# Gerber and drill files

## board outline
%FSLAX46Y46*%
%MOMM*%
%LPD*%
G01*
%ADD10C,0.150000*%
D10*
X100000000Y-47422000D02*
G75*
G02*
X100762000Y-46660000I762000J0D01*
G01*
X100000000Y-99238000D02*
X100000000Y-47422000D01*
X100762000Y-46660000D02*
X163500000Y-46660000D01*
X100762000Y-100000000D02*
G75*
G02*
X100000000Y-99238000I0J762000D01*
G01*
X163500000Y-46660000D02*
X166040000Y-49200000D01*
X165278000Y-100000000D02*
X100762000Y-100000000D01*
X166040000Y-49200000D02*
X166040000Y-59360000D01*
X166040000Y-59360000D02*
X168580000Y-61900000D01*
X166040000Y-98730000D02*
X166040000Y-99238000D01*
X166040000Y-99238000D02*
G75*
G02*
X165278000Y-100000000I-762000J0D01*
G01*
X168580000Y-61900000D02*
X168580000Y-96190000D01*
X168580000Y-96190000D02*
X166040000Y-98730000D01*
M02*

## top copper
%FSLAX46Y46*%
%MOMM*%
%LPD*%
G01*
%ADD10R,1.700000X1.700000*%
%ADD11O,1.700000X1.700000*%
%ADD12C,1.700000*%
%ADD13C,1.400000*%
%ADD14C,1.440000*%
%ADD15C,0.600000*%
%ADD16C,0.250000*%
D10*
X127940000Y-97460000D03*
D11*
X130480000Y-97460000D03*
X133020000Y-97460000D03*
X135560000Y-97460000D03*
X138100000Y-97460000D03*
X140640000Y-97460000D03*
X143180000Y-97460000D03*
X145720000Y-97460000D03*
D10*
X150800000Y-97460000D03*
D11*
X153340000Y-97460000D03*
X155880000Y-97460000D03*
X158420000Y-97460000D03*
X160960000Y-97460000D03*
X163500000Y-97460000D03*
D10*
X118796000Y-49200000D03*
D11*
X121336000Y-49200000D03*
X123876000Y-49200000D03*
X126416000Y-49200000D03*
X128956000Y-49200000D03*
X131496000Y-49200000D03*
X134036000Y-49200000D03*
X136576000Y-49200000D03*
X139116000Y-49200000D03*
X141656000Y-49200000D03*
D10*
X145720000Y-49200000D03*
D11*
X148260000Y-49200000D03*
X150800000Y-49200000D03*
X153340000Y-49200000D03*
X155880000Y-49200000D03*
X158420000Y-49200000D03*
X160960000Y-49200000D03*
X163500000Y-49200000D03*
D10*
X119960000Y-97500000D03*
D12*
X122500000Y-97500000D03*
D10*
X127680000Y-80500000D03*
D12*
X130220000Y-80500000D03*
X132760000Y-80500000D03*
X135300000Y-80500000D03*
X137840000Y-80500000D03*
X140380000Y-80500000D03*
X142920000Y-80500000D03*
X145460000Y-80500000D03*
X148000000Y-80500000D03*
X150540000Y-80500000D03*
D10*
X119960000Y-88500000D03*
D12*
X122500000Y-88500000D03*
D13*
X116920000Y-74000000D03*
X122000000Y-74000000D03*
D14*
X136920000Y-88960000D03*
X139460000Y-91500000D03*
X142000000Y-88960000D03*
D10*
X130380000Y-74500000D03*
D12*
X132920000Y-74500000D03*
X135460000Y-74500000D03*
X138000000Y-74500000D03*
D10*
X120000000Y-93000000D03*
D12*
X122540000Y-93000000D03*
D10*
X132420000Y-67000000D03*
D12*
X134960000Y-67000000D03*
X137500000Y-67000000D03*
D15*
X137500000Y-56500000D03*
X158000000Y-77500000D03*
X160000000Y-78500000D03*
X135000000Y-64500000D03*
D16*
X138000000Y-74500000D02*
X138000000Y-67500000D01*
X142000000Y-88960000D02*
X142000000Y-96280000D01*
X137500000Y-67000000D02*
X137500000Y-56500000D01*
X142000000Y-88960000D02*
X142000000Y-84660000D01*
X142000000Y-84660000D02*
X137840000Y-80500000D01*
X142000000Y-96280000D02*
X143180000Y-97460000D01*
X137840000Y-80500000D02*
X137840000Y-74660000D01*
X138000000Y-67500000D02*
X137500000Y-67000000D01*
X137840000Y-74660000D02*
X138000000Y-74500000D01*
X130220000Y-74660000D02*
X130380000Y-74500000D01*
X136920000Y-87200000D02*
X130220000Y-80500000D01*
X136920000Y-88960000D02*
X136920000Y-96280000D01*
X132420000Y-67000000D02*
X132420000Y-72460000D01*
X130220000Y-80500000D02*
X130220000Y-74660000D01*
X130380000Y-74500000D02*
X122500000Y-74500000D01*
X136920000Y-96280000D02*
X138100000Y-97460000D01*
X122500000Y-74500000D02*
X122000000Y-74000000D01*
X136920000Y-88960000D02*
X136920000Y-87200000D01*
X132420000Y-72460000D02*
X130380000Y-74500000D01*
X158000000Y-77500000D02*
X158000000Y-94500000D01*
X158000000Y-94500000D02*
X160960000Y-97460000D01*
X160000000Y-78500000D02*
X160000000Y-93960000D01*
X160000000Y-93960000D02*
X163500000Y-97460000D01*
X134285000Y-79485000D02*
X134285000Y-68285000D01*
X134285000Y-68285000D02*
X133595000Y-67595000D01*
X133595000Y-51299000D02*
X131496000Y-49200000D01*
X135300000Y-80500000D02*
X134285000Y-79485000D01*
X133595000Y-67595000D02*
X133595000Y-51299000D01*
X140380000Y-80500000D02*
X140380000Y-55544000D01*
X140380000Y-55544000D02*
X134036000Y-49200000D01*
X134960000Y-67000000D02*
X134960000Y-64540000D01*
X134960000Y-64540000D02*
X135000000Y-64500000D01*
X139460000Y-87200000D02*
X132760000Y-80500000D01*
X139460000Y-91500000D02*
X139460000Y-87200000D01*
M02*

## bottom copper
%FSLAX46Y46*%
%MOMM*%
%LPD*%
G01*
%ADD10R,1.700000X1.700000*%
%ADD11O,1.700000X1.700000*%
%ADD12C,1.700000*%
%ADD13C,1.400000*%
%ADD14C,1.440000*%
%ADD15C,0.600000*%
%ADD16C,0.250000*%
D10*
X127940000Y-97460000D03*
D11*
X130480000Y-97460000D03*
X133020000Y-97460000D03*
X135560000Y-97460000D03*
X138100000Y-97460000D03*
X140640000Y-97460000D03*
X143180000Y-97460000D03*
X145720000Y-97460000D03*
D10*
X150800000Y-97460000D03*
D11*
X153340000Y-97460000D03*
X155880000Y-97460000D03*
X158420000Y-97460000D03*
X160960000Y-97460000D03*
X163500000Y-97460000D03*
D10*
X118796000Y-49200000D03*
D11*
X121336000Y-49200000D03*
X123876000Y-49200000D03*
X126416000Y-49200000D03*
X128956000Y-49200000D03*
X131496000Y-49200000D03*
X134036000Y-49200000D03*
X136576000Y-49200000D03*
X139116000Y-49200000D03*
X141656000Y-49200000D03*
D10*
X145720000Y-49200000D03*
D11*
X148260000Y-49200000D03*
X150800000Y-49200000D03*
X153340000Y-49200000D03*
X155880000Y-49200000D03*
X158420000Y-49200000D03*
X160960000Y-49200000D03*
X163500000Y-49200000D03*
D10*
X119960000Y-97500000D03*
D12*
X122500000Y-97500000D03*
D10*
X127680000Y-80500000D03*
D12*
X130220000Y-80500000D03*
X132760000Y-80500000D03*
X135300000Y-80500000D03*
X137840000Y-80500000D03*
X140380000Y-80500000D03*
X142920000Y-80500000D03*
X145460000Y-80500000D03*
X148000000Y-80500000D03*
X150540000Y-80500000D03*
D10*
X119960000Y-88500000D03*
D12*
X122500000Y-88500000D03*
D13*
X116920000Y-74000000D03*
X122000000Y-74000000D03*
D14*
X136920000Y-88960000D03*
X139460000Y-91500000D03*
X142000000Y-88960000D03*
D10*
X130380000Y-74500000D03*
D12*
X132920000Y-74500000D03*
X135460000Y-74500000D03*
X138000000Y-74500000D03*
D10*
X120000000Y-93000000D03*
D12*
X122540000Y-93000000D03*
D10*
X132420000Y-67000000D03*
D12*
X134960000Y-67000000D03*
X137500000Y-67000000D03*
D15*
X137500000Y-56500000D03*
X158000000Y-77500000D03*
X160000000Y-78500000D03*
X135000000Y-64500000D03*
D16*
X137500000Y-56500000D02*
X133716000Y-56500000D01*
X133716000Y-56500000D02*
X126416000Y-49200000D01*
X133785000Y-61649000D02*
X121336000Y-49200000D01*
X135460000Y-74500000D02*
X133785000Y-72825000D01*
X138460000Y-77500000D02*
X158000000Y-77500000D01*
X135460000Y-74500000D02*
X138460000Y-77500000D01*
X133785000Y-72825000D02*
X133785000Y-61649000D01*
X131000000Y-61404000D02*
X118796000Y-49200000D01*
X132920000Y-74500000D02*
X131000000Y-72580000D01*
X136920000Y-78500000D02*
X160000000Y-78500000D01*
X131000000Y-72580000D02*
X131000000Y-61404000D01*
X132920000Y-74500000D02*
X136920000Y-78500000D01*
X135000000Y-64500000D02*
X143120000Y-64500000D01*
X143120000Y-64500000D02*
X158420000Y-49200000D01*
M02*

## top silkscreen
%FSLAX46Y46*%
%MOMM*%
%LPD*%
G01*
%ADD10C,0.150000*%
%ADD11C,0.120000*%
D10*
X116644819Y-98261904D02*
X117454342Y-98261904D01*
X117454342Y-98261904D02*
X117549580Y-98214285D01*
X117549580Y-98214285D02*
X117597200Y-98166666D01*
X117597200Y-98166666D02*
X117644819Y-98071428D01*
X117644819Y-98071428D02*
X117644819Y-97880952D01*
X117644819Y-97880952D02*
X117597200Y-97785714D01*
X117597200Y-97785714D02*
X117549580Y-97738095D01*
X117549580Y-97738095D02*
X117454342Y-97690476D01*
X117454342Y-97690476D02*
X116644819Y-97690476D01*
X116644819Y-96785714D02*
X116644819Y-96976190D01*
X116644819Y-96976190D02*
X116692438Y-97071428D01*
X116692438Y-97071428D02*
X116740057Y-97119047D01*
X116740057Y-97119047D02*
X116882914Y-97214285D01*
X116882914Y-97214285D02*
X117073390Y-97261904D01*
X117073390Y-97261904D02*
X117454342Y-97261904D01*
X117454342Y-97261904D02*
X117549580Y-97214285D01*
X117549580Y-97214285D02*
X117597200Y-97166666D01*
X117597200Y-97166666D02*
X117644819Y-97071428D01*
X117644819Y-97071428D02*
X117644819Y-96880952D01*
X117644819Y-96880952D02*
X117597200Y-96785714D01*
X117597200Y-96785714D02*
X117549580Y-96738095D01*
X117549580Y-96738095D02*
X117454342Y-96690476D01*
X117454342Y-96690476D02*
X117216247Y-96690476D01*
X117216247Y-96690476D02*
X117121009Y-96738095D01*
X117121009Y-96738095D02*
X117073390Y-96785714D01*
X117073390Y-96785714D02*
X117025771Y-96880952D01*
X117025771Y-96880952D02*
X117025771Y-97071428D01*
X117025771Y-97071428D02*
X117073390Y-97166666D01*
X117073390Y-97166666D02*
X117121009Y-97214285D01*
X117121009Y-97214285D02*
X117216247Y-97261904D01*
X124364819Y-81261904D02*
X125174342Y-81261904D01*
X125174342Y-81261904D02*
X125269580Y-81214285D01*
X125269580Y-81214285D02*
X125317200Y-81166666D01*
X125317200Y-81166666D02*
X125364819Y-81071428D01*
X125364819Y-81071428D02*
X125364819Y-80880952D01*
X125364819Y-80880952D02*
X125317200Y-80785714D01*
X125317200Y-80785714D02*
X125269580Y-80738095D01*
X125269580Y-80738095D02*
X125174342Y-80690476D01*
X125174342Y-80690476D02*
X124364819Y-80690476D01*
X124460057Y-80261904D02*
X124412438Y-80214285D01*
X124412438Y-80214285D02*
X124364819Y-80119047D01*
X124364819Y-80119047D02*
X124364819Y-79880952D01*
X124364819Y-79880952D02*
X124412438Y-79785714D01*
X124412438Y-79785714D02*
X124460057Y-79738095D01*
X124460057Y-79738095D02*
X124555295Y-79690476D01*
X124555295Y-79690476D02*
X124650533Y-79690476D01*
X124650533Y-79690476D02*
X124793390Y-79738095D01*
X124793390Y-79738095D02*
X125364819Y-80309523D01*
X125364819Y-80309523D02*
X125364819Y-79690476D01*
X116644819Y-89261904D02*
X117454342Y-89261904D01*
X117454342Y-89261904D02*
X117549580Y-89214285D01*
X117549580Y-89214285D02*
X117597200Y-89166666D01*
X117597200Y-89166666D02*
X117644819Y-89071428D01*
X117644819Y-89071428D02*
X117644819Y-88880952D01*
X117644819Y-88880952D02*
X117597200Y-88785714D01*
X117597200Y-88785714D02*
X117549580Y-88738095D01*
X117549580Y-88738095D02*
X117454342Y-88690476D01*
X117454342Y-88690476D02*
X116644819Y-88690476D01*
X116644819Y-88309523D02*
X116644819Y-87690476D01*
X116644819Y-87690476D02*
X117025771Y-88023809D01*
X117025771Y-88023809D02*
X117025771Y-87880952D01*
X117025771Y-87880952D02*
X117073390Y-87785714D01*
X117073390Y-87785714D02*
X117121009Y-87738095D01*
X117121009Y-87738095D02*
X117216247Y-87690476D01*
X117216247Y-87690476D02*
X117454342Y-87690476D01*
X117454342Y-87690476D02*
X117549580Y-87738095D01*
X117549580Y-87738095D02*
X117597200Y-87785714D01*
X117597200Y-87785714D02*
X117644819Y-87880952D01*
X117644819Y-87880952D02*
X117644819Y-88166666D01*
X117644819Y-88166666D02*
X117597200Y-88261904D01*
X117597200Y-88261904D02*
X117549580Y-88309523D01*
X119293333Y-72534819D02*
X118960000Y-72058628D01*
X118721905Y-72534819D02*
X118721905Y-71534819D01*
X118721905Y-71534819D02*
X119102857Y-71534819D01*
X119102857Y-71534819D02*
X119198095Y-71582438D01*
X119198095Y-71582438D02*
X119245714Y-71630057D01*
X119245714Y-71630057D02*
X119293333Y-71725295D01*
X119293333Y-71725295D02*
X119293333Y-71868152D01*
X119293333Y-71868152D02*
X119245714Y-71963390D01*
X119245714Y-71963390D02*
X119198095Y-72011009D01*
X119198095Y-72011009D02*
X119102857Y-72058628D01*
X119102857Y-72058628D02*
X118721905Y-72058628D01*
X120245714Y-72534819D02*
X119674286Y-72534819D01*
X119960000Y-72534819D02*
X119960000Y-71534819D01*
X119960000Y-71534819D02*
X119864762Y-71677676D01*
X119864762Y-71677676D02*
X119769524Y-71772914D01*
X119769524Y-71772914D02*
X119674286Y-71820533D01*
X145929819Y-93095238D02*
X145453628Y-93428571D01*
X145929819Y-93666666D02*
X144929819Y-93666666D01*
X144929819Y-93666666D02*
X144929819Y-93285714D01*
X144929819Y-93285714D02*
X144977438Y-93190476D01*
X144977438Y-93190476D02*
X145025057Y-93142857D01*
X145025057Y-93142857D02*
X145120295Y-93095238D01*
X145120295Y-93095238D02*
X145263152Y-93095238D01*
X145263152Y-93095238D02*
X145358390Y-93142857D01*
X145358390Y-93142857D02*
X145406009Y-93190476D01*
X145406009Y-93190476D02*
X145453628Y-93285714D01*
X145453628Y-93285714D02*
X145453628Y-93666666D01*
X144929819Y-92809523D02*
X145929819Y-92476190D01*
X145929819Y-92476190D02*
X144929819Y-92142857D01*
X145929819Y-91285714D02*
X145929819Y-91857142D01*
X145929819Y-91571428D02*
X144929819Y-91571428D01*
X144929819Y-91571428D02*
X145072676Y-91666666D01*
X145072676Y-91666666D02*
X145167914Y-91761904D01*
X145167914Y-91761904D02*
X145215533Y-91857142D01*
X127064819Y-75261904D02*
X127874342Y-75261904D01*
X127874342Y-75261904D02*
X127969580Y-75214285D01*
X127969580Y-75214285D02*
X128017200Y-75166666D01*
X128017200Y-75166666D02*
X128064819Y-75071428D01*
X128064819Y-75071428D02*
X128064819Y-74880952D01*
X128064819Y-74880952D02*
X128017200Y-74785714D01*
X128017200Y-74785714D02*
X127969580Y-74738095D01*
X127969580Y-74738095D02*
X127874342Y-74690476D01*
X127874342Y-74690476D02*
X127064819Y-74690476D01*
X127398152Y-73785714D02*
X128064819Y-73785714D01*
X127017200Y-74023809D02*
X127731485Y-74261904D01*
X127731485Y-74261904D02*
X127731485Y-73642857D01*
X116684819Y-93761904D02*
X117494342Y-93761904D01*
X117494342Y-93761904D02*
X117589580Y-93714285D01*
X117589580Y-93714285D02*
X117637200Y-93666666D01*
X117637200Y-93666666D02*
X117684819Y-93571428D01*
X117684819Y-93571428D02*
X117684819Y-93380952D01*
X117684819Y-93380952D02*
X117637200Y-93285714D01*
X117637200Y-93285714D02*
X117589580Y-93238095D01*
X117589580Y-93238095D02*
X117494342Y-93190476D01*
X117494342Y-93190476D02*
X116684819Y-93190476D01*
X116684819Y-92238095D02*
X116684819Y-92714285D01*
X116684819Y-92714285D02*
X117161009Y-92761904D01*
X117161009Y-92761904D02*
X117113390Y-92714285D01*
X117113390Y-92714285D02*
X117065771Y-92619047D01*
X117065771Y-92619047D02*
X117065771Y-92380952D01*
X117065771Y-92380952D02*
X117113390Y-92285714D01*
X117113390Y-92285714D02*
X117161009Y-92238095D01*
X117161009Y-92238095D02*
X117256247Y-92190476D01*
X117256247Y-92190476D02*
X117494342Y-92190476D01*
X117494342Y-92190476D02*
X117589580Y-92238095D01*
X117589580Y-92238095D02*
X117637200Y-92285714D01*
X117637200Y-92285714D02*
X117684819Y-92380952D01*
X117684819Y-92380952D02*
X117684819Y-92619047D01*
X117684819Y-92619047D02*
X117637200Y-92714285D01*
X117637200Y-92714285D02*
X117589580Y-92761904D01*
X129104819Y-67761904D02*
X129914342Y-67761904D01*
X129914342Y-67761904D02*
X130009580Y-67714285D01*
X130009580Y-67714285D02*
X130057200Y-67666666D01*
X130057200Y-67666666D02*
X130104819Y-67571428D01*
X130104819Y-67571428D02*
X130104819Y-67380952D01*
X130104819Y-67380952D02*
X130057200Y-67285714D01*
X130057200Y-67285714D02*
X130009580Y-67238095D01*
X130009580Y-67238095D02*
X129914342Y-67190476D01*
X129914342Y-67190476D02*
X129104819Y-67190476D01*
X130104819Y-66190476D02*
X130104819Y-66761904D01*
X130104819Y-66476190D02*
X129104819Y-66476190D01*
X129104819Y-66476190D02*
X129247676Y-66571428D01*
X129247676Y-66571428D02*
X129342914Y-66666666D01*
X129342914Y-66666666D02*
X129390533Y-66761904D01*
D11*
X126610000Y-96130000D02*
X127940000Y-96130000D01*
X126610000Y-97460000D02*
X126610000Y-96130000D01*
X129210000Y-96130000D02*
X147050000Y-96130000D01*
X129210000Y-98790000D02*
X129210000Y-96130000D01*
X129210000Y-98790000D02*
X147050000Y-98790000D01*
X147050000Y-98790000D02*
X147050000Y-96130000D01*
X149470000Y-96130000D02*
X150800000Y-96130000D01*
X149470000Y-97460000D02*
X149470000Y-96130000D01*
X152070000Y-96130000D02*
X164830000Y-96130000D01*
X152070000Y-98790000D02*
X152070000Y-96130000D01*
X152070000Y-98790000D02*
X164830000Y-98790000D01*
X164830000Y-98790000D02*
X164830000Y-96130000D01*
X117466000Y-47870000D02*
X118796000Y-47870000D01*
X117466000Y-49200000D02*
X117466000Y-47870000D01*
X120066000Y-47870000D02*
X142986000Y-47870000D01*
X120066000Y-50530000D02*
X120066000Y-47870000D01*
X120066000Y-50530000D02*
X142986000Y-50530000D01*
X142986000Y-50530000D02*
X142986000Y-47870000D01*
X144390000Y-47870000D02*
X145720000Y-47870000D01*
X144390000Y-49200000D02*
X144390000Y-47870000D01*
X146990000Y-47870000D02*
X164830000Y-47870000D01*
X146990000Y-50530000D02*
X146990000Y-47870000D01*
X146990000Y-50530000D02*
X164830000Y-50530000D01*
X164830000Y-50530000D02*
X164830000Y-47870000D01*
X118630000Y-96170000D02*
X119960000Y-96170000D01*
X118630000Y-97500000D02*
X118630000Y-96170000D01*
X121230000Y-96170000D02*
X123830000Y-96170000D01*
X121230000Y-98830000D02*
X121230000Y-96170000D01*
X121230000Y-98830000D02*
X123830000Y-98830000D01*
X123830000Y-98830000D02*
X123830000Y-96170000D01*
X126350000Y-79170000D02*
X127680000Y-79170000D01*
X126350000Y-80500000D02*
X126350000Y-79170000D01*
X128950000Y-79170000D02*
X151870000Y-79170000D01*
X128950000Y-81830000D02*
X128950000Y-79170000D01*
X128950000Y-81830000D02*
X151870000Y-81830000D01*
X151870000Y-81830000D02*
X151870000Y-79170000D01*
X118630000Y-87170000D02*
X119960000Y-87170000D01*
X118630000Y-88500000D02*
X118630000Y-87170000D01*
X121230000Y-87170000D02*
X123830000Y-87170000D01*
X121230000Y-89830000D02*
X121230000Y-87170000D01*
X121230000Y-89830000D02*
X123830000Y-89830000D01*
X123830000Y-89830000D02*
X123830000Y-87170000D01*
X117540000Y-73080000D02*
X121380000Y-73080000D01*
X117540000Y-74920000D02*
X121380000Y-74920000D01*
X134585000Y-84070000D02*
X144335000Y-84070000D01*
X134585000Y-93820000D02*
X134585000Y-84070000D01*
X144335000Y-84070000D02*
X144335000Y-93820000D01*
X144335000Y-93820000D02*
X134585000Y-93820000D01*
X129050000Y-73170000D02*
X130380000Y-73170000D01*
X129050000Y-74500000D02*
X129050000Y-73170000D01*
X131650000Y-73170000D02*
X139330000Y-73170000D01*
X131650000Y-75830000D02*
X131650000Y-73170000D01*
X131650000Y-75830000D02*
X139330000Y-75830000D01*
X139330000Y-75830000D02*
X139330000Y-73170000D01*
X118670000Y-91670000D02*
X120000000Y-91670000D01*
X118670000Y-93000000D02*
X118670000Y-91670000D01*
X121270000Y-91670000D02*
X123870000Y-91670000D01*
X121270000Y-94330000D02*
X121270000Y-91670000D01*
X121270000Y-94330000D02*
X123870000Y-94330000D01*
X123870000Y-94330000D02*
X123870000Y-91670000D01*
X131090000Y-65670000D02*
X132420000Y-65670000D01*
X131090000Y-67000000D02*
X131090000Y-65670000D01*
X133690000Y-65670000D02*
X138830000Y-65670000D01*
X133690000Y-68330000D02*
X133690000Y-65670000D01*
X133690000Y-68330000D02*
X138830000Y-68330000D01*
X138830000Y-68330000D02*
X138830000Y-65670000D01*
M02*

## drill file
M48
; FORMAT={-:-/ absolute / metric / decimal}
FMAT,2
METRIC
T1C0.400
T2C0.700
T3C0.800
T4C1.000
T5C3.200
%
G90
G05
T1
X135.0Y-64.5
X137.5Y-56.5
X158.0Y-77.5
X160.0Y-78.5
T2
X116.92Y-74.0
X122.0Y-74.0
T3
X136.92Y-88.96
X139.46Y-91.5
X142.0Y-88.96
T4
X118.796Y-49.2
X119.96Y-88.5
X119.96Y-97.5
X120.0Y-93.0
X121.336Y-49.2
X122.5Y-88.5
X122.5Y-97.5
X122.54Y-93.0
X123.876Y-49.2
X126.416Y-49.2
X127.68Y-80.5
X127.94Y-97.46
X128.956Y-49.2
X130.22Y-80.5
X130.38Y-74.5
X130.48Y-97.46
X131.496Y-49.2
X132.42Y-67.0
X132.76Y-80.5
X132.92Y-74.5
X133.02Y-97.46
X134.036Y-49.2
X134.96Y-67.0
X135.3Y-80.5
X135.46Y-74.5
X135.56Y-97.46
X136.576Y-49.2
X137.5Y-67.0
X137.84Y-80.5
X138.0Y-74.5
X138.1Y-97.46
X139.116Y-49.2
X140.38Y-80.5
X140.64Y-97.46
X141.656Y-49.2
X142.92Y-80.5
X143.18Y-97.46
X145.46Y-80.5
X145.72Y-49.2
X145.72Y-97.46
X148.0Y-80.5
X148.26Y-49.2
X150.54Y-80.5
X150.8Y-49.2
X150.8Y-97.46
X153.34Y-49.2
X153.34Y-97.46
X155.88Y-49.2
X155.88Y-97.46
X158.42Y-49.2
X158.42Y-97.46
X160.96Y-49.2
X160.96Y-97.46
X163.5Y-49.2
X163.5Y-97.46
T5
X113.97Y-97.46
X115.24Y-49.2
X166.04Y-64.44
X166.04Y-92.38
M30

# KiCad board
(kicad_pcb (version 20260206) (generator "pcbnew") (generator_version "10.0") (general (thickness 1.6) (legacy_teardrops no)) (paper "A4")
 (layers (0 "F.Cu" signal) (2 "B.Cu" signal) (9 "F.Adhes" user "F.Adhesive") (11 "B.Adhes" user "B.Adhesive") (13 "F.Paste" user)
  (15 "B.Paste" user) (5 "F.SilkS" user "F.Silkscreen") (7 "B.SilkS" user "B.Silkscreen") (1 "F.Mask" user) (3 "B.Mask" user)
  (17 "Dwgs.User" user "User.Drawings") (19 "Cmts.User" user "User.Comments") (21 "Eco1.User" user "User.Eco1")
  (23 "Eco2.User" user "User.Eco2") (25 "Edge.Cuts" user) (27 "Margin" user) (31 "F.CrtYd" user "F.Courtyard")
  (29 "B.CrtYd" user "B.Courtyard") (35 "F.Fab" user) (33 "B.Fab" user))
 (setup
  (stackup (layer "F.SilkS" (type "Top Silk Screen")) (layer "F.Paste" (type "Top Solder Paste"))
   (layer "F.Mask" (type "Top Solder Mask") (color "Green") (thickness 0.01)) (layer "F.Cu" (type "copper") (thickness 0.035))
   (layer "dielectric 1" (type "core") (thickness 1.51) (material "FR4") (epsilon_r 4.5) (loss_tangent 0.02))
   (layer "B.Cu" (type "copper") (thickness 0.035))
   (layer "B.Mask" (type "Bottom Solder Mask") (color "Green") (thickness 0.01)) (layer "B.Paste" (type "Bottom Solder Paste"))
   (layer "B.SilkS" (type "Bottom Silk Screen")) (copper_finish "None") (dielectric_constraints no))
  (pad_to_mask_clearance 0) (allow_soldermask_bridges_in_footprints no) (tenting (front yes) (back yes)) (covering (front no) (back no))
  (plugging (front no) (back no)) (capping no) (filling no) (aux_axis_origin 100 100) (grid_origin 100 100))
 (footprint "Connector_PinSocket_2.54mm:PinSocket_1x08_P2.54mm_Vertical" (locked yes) (layer "F.Cu") (at 127.94 97.46 90)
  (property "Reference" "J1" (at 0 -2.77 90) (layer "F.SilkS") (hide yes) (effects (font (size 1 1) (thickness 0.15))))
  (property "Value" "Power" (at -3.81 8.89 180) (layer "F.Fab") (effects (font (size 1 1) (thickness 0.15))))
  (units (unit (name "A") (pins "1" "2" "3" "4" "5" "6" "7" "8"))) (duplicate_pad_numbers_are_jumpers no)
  (fp_line (start 1.33 -1.33) (end 1.33 0) (stroke (width 0.12) (type solid)) (layer "F.SilkS"))
  (fp_line (start 0 -1.33) (end 1.33 -1.33) (stroke (width 0.12) (type solid)) (layer "F.SilkS"))
  (fp_line (start 1.33 1.27) (end 1.33 19.11) (stroke (width 0.12) (type solid)) (layer "F.SilkS"))
  (fp_line (start -1.33 1.27) (end 1.33 1.27) (stroke (width 0.12) (type solid)) (layer "F.SilkS"))
  (fp_line (start -1.33 1.27) (end -1.33 19.11) (stroke (width 0.12) (type solid)) (layer "F.SilkS"))
  (fp_line (start -1.33 19.11) (end 1.33 19.11) (stroke (width 0.12) (type solid)) (layer "F.SilkS"))
  (pad "1" thru_hole rect (at 0 0 90) (size 1.7 1.7) (drill 1) (layers "*.Cu" "*.Mask") (remove_unused_layers no)
   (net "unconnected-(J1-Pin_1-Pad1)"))
  (pad "2" thru_hole oval (at 0 2.54 90) (size 1.7 1.7) (drill 1) (layers "*.Cu" "*.Mask") (remove_unused_layers no) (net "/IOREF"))
  (pad "3" thru_hole oval (at 0 5.08 90) (size 1.7 1.7) (drill 1) (layers "*.Cu" "*.Mask") (remove_unused_layers no) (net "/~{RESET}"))
  (pad "4" thru_hole oval (at 0 7.62 90) (size 1.7 1.7) (drill 1) (layers "*.Cu" "*.Mask") (remove_unused_layers no) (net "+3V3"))
  (pad "5" thru_hole oval (at 0 10.16 90) (size 1.7 1.7) (drill 1) (layers "*.Cu" "*.Mask") (remove_unused_layers no) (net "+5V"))
  (pad "6" thru_hole oval (at 0 12.7 90) (size 1.7 1.7) (drill 1) (layers "*.Cu" "*.Mask") (remove_unused_layers no) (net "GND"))
  (pad "7" thru_hole oval (at 0 15.24 90) (size 1.7 1.7) (drill 1) (layers "*.Cu" "*.Mask") (remove_unused_layers no) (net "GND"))
  (pad "8" thru_hole oval (at 0 17.78 90) (size 1.7 1.7) (drill 1) (layers "*.Cu" "*.Mask") (remove_unused_layers no) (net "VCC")))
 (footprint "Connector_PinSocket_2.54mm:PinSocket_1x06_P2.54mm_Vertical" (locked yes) (layer "F.Cu") (at 150.8 97.46 90)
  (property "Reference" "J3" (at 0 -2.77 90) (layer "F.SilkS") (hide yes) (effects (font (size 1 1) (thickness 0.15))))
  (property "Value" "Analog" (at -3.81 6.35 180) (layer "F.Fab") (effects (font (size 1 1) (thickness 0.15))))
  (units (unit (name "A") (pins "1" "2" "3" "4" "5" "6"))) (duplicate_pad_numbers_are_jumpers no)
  (fp_line (start 1.33 -1.33) (end 1.33 0) (stroke (width 0.12) (type solid)) (layer "F.SilkS"))
  (fp_line (start 0 -1.33) (end 1.33 -1.33) (stroke (width 0.12) (type solid)) (layer "F.SilkS"))
  (fp_line (start 1.33 1.27) (end 1.33 14.03) (stroke (width 0.12) (type solid)) (layer "F.SilkS"))
  (fp_line (start -1.33 1.27) (end 1.33 1.27) (stroke (width 0.12) (type solid)) (layer "F.SilkS"))
  (fp_line (start -1.33 1.27) (end -1.33 14.03) (stroke (width 0.12) (type solid)) (layer "F.SilkS"))
  (fp_line (start -1.33 14.03) (end 1.33 14.03) (stroke (width 0.12) (type solid)) (layer "F.SilkS"))
  (pad "1" thru_hole rect (at 0 0 90) (size 1.7 1.7) (drill 1) (layers "*.Cu" "*.Mask") (remove_unused_layers no) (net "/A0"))
  (pad "2" thru_hole oval (at 0 2.54 90) (size 1.7 1.7) (drill 1) (layers "*.Cu" "*.Mask") (remove_unused_layers no) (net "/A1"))
  (pad "3" thru_hole oval (at 0 5.08 90) (size 1.7 1.7) (drill 1) (layers "*.Cu" "*.Mask") (remove_unused_layers no) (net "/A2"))
  (pad "4" thru_hole oval (at 0 7.62 90) (size 1.7 1.7) (drill 1) (layers "*.Cu" "*.Mask") (remove_unused_layers no) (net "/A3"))
  (pad "5" thru_hole oval (at 0 10.16 90) (size 1.7 1.7) (drill 1) (layers "*.Cu" "*.Mask") (remove_unused_layers no) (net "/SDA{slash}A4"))
  (pad "6" thru_hole oval (at 0 12.7 90) (size 1.7 1.7) (drill 1) (layers "*.Cu" "*.Mask") (remove_unused_layers no) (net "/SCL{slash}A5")))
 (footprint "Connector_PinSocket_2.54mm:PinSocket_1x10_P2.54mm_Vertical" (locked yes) (layer "F.Cu") (at 118.796 49.2 90)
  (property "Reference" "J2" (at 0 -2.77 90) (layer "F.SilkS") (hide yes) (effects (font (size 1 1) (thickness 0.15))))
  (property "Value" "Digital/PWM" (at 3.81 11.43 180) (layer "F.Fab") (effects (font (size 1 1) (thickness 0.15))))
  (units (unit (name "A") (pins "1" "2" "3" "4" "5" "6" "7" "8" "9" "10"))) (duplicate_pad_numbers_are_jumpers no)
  (fp_line (start 1.33 -1.33) (end 1.33 0) (stroke (width 0.12) (type solid)) (layer "F.SilkS"))
  (fp_line (start 0 -1.33) (end 1.33 -1.33) (stroke (width 0.12) (type solid)) (layer "F.SilkS"))
  (fp_line (start 1.33 1.27) (end 1.33 24.19) (stroke (width 0.12) (type solid)) (layer "F.SilkS"))
  (fp_line (start -1.33 1.27) (end 1.33 1.27) (stroke (width 0.12) (type solid)) (layer "F.SilkS"))
  (fp_line (start -1.33 1.27) (end -1.33 24.19) (stroke (width 0.12) (type solid)) (layer "F.SilkS"))
  (fp_line (start -1.33 24.19) (end 1.33 24.19) (stroke (width 0.12) (type solid)) (layer "F.SilkS"))
  (pad "1" thru_hole rect (at 0 0 90) (size 1.7 1.7) (drill 1) (layers "*.Cu" "*.Mask") (remove_unused_layers no) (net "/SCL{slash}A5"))
  (pad "2" thru_hole oval (at 0 2.54 90) (size 1.7 1.7) (drill 1) (layers "*.Cu" "*.Mask") (remove_unused_layers no) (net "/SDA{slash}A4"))
  (pad "3" thru_hole oval (at 0 5.08 90) (size 1.7 1.7) (drill 1) (layers "*.Cu" "*.Mask") (remove_unused_layers no) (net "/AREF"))
  (pad "4" thru_hole oval (at 0 7.62 90) (size 1.7 1.7) (drill 1) (layers "*.Cu" "*.Mask") (remove_unused_layers no) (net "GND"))
  (pad "5" thru_hole oval (at 0 10.16 90) (size 1.7 1.7) (drill 1) (layers "*.Cu" "*.Mask") (remove_unused_layers no) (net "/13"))
  (pad "6" thru_hole oval (at 0 12.7 90) (size 1.7 1.7) (drill 1) (layers "*.Cu" "*.Mask") (remove_unused_layers no) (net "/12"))
  (pad "7" thru_hole oval (at 0 15.24 90) (size 1.7 1.7) (drill 1) (layers "*.Cu" "*.Mask") (remove_unused_layers no) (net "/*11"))
  (pad "8" thru_hole oval (at 0 17.78 90) (size 1.7 1.7) (drill 1) (layers "*.Cu" "*.Mask") (remove_unused_layers no) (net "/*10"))
  (pad "9" thru_hole oval (at 0 20.32 90) (size 1.7 1.7) (drill 1) (layers "*.Cu" "*.Mask") (remove_unused_layers no) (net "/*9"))
  (pad "10" thru_hole oval (at 0 22.86 90) (size 1.7 1.7) (drill 1) (layers "*.Cu" "*.Mask") (remove_unused_layers no) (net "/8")))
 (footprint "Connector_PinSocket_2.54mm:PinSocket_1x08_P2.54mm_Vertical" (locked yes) (layer "F.Cu") (at 145.72 49.2 90)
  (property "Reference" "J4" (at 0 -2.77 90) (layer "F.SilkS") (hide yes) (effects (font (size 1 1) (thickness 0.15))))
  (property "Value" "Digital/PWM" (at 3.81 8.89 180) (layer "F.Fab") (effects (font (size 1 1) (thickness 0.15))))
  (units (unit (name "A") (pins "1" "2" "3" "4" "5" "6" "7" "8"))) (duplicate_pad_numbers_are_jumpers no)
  (fp_line (start 1.33 -1.33) (end 1.33 0) (stroke (width 0.12) (type solid)) (layer "F.SilkS"))
  (fp_line (start 0 -1.33) (end 1.33 -1.33) (stroke (width 0.12) (type solid)) (layer "F.SilkS"))
  (fp_line (start 1.33 1.27) (end 1.33 19.11) (stroke (width 0.12) (type solid)) (layer "F.SilkS"))
  (fp_line (start -1.33 1.27) (end 1.33 1.27) (stroke (width 0.12) (type solid)) (layer "F.SilkS"))
  (fp_line (start -1.33 1.27) (end -1.33 19.11) (stroke (width 0.12) (type solid)) (layer "F.SilkS"))
  (fp_line (start -1.33 19.11) (end 1.33 19.11) (stroke (width 0.12) (type solid)) (layer "F.SilkS"))
  (pad "1" thru_hole rect (at 0 0 90) (size 1.7 1.7) (drill 1) (layers "*.Cu" "*.Mask") (remove_unused_layers no) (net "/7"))
  (pad "2" thru_hole oval (at 0 2.54 90) (size 1.7 1.7) (drill 1) (layers "*.Cu" "*.Mask") (remove_unused_layers no) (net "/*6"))
  (pad "3" thru_hole oval (at 0 5.08 90) (size 1.7 1.7) (drill 1) (layers "*.Cu" "*.Mask") (remove_unused_layers no) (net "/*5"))
  (pad "4" thru_hole oval (at 0 7.62 90) (size 1.7 1.7) (drill 1) (layers "*.Cu" "*.Mask") (remove_unused_layers no) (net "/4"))
  (pad "5" thru_hole oval (at 0 10.16 90) (size 1.7 1.7) (drill 1) (layers "*.Cu" "*.Mask") (remove_unused_layers no) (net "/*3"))
  (pad "6" thru_hole oval (at 0 12.7 90) (size 1.7 1.7) (drill 1) (layers "*.Cu" "*.Mask") (remove_unused_layers no) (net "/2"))
  (pad "7" thru_hole oval (at 0 15.24 90) (size 1.7 1.7) (drill 1) (layers "*.Cu" "*.Mask") (remove_unused_layers no) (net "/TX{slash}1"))
  (pad "8" thru_hole oval (at 0 17.78 90) (size 1.7 1.7) (drill 1) (layers "*.Cu" "*.Mask") (remove_unused_layers no) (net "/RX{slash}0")))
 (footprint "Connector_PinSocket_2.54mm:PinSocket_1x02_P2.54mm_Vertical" (layer "F.Cu") (at 119.96 97.5 90)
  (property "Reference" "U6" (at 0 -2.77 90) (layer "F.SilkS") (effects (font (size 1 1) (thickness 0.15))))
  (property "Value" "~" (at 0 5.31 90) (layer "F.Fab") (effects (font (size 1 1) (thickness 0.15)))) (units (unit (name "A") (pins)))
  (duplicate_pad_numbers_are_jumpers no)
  (fp_line (start 1.33 -1.33) (end 1.33 0) (stroke (width 0.12) (type solid)) (layer "F.SilkS"))
  (fp_line (start 0 -1.33) (end 1.33 -1.33) (stroke (width 0.12) (type solid)) (layer "F.SilkS"))
  (fp_line (start 1.33 1.27) (end 1.33 3.87) (stroke (width 0.12) (type solid)) (layer "F.SilkS"))
  (fp_line (start -1.33 1.27) (end 1.33 1.27) (stroke (width 0.12) (type solid)) (layer "F.SilkS"))
  (fp_line (start -1.33 1.27) (end -1.33 3.87) (stroke (width 0.12) (type solid)) (layer "F.SilkS"))
  (fp_line (start -1.33 3.87) (end 1.33 3.87) (stroke (width 0.12) (type solid)) (layer "F.SilkS"))
  (pad "1" thru_hole rect (at 0 0 90) (size 1.7 1.7) (drill 1) (layers "*.Cu" "*.Mask") (remove_unused_layers no))
  (pad "2" thru_hole circle (at 0 2.54 90) (size 1.7 1.7) (drill 1) (layers "*.Cu" "*.Mask") (remove_unused_layers no)))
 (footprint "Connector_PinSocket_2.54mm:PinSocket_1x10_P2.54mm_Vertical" (layer "F.Cu") (at 127.68 80.5 90)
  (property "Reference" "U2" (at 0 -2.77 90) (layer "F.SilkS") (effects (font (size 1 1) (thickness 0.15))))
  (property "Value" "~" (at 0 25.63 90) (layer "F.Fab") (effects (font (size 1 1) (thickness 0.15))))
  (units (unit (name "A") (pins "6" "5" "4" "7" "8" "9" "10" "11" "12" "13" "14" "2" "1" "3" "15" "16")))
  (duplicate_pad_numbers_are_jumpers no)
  (fp_line (start 1.33 -1.33) (end 1.33 0) (stroke (width 0.12) (type solid)) (layer "F.SilkS"))
  (fp_line (start 0 -1.33) (end 1.33 -1.33) (stroke (width 0.12) (type solid)) (layer "F.SilkS"))
  (fp_line (start 1.33 1.27) (end 1.33 24.19) (stroke (width 0.12) (type solid)) (layer "F.SilkS"))
  (fp_line (start -1.33 1.27) (end 1.33 1.27) (stroke (width 0.12) (type solid)) (layer "F.SilkS"))
  (fp_line (start -1.33 1.27) (end -1.33 24.19) (stroke (width 0.12) (type solid)) (layer "F.SilkS"))
  (fp_line (start -1.33 24.19) (end 1.33 24.19) (stroke (width 0.12) (type solid)) (layer "F.SilkS"))
  (pad "1" thru_hole rect (at 0 0 90) (size 1.7 1.7) (drill 1) (layers "*.Cu" "*.Mask") (remove_unused_layers no) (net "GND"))
  (pad "2" thru_hole circle (at 0 2.54 90) (size 1.7 1.7) (drill 1) (layers "*.Cu" "*.Mask") (remove_unused_layers no) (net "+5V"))
  (pad "3" thru_hole circle (at 0 5.08 90) (size 1.7 1.7) (drill 1) (layers "*.Cu" "*.Mask") (remove_unused_layers no) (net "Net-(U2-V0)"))
  (pad "4" thru_hole circle (at 0 7.62 90) (size 1.7 1.7) (drill 1) (layers "*.Cu" "*.Mask") (remove_unused_layers no) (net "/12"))
  (pad "5" thru_hole circle (at 0 10.16 90) (size 1.7 1.7) (drill 1) (layers "*.Cu" "*.Mask") (remove_unused_layers no) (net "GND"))
  (pad "6" thru_hole circle (at 0 12.7 90) (size 1.7 1.7) (drill 1) (layers "*.Cu" "*.Mask") (remove_unused_layers no) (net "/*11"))
  (pad "7" thru_hole circle (at 0 15.24 90) (size 1.7 1.7) (drill 1) (layers "*.Cu" "*.Mask") (remove_unused_layers no)
   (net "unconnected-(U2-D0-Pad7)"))
  (pad "8" thru_hole circle (at 0 17.78 90) (size 1.7 1.7) (drill 1) (layers "*.Cu" "*.Mask") (remove_unused_layers no)
   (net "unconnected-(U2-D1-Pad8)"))
  (pad "9" thru_hole circle (at 0 20.32 90) (size 1.7 1.7) (drill 1) (layers "*.Cu" "*.Mask") (remove_unused_layers no)
   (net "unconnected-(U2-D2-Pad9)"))
  (pad "10" thru_hole circle (at 0 22.86 90) (size 1.7 1.7) (drill 1) (layers "*.Cu" "*.Mask") (remove_unused_layers no)
   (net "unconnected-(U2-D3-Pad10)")))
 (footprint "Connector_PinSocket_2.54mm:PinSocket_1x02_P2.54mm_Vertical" (layer "F.Cu") (at 119.96 88.5 90)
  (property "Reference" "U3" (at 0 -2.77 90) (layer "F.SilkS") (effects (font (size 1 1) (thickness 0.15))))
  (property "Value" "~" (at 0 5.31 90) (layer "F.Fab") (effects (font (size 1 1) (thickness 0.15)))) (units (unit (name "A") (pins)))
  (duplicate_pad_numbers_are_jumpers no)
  (fp_line (start 1.33 -1.33) (end 1.33 0) (stroke (width 0.12) (type solid)) (layer "F.SilkS"))
  (fp_line (start 0 -1.33) (end 1.33 -1.33) (stroke (width 0.12) (type solid)) (layer "F.SilkS"))
  (fp_line (start 1.33 1.27) (end 1.33 3.87) (stroke (width 0.12) (type solid)) (layer "F.SilkS"))
  (fp_line (start -1.33 1.27) (end 1.33 1.27) (stroke (width 0.12) (type solid)) (layer "F.SilkS"))
  (fp_line (start -1.33 1.27) (end -1.33 3.87) (stroke (width 0.12) (type solid)) (layer "F.SilkS"))
  (fp_line (start -1.33 3.87) (end 1.33 3.87) (stroke (width 0.12) (type solid)) (layer "F.SilkS"))
  (pad "1" thru_hole rect (at 0 0 90) (size 1.7 1.7) (drill 1) (layers "*.Cu" "*.Mask") (remove_unused_layers no))
  (pad "2" thru_hole circle (at 0 2.54 90) (size 1.7 1.7) (drill 1) (layers "*.Cu" "*.Mask") (remove_unused_layers no)))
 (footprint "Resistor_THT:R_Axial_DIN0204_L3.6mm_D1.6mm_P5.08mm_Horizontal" (layer "F.Cu") (at 116.92 74)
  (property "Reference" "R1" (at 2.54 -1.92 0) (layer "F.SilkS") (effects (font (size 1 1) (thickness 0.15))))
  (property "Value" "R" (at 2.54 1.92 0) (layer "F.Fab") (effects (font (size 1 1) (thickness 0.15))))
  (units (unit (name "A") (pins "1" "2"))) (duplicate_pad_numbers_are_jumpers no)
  (fp_line (start 0.62 -0.92) (end 4.46 -0.92) (stroke (width 0.12) (type solid)) (layer "F.SilkS"))
  (fp_line (start 0.62 0.92) (end 4.46 0.92) (stroke (width 0.12) (type solid)) (layer "F.SilkS"))
  (pad "1" thru_hole circle (at 0 0) (size 1.4 1.4) (drill 0.7) (layers "*.Cu" "*.Mask") (remove_unused_layers no) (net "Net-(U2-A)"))
  (pad "2" thru_hole circle (at 5.08 0) (size 1.4 1.4) (drill 0.7) (layers "*.Cu" "*.Mask") (remove_unused_layers no) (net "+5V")))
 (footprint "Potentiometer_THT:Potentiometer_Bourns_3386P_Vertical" (layer "F.Cu") (at 136.92 88.96 -90)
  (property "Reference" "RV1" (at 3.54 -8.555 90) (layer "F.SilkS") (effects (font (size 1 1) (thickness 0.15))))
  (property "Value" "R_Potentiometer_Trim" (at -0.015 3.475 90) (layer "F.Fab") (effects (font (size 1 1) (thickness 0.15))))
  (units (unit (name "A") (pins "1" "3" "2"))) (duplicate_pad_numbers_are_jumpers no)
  (fp_line (start -4.89 2.335) (end -4.89 -7.415) (stroke (width 0.12) (type solid)) (layer "F.SilkS"))
  (fp_line (start 4.86 2.335) (end -4.89 2.335) (stroke (width 0.12) (type solid)) (layer "F.SilkS"))
  (fp_line (start -4.89 -7.415) (end 4.86 -7.415) (stroke (width 0.12) (type solid)) (layer "F.SilkS"))
  (fp_line (start 4.86 -7.415) (end 4.86 2.335) (stroke (width 0.12) (type solid)) (layer "F.SilkS"))
  (pad "1" thru_hole circle (at 0 0 270) (size 1.44 1.44) (drill 0.8) (layers "*.Cu" "*.Mask") (remove_unused_layers no) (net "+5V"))
  (pad "2" thru_hole circle (at 2.54 -2.54 270) (size 1.44 1.44) (drill 0.8) (layers "*.Cu" "*.Mask") (remove_unused_layers no)
   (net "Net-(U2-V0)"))
  (pad "3" thru_hole circle (at 0 -5.08 270) (size 1.44 1.44) (drill 0.8) (layers "*.Cu" "*.Mask") (remove_unused_layers no) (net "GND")))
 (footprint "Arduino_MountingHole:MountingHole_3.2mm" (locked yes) (layer "F.Cu") (at 115.24 49.2)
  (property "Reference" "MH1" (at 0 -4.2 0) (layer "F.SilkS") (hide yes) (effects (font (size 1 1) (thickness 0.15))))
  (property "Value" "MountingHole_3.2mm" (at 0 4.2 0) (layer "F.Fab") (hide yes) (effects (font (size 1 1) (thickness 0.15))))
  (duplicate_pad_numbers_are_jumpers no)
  (pad "" np_thru_hole circle (at 0 0) (size 3.2 3.2) (drill 3.2) (layers "*.Cu" "*.Mask")))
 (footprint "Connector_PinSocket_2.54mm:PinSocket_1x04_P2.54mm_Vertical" (layer "F.Cu") (at 130.38 74.5 90)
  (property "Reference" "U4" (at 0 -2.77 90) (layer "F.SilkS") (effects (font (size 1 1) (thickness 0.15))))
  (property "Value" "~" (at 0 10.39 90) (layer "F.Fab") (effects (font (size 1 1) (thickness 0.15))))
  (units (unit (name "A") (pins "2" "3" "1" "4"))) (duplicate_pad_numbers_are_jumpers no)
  (fp_line (start 1.33 -1.33) (end 1.33 0) (stroke (width 0.12) (type solid)) (layer "F.SilkS"))
  (fp_line (start 0 -1.33) (end 1.33 -1.33) (stroke (width 0.12) (type solid)) (layer "F.SilkS"))
  (fp_line (start 1.33 1.27) (end 1.33 8.95) (stroke (width 0.12) (type solid)) (layer "F.SilkS"))
  (fp_line (start -1.33 1.27) (end 1.33 1.27) (stroke (width 0.12) (type solid)) (layer "F.SilkS"))
  (fp_line (start -1.33 1.27) (end -1.33 8.95) (stroke (width 0.12) (type solid)) (layer "F.SilkS"))
  (fp_line (start -1.33 8.95) (end 1.33 8.95) (stroke (width 0.12) (type solid)) (layer "F.SilkS"))
  (pad "1" thru_hole rect (at 0 0 90) (size 1.7 1.7) (drill 1) (layers "*.Cu" "*.Mask") (remove_unused_layers no) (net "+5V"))
  (pad "2" thru_hole circle (at 0 2.54 90) (size 1.7 1.7) (drill 1) (layers "*.Cu" "*.Mask") (remove_unused_layers no) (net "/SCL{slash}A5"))
  (pad "3" thru_hole circle (at 0 5.08 90) (size 1.7 1.7) (drill 1) (layers "*.Cu" "*.Mask") (remove_unused_layers no) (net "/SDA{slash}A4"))
  (pad "4" thru_hole circle (at 0 7.62 90) (size 1.7 1.7) (drill 1) (layers "*.Cu" "*.Mask") (remove_unused_layers no) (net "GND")))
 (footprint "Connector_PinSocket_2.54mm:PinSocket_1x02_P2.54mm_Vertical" (layer "F.Cu") (at 120 93 90)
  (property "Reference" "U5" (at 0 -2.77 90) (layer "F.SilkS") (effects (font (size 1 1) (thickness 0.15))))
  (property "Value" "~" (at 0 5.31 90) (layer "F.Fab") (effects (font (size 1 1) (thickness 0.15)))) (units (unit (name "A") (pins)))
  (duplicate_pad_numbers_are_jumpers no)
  (fp_line (start 1.33 -1.33) (end 1.33 0) (stroke (width 0.12) (type solid)) (layer "F.SilkS"))
  (fp_line (start 0 -1.33) (end 1.33 -1.33) (stroke (width 0.12) (type solid)) (layer "F.SilkS"))
  (fp_line (start 1.33 1.27) (end 1.33 3.87) (stroke (width 0.12) (type solid)) (layer "F.SilkS"))
  (fp_line (start -1.33 1.27) (end 1.33 1.27) (stroke (width 0.12) (type solid)) (layer "F.SilkS"))
  (fp_line (start -1.33 1.27) (end -1.33 3.87) (stroke (width 0.12) (type solid)) (layer "F.SilkS"))
  (fp_line (start -1.33 3.87) (end 1.33 3.87) (stroke (width 0.12) (type solid)) (layer "F.SilkS"))
  (pad "1" thru_hole rect (at 0 0 90) (size 1.7 1.7) (drill 1) (layers "*.Cu" "*.Mask") (remove_unused_layers no))
  (pad "2" thru_hole circle (at 0 2.54 90) (size 1.7 1.7) (drill 1) (layers "*.Cu" "*.Mask") (remove_unused_layers no)))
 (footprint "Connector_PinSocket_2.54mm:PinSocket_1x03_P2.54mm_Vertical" (layer "F.Cu") (at 132.42 67 90)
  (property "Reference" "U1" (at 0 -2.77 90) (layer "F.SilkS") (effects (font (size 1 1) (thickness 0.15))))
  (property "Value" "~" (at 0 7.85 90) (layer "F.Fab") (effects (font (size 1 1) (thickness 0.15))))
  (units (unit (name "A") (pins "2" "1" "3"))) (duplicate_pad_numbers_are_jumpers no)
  (fp_line (start 1.33 -1.33) (end 1.33 0) (stroke (width 0.12) (type solid)) (layer "F.SilkS"))
  (fp_line (start 0 -1.33) (end 1.33 -1.33) (stroke (width 0.12) (type solid)) (layer "F.SilkS"))
  (fp_line (start 1.33 1.27) (end 1.33 6.41) (stroke (width 0.12) (type solid)) (layer "F.SilkS"))
  (fp_line (start -1.33 1.27) (end 1.33 1.27) (stroke (width 0.12) (type solid)) (layer "F.SilkS"))
  (fp_line (start -1.33 1.27) (end -1.33 6.41) (stroke (width 0.12) (type solid)) (layer "F.SilkS"))
  (fp_line (start -1.33 6.41) (end 1.33 6.41) (stroke (width 0.12) (type solid)) (layer "F.SilkS"))
  (pad "1" thru_hole rect (at 0 0 90) (size 1.7 1.7) (drill 1) (layers "*.Cu" "*.Mask") (remove_unused_layers no) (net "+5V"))
  (pad "2" thru_hole circle (at 0 2.54 90) (size 1.7 1.7) (drill 1) (layers "*.Cu" "*.Mask") (remove_unused_layers no) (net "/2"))
  (pad "3" thru_hole circle (at 0 5.08 90) (size 1.7 1.7) (drill 1) (layers "*.Cu" "*.Mask") (remove_unused_layers no) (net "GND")))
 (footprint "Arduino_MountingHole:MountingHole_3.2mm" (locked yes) (layer "F.Cu") (at 113.97 97.46)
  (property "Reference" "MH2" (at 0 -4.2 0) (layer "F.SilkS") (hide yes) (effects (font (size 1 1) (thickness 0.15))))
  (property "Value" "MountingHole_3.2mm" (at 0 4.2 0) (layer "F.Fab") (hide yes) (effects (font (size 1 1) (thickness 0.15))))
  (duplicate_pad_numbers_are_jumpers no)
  (pad "" np_thru_hole circle (at 0 0) (size 3.2 3.2) (drill 3.2) (layers "*.Cu" "*.Mask")))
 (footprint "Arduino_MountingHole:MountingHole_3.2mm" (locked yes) (layer "F.Cu") (at 166.04 64.44)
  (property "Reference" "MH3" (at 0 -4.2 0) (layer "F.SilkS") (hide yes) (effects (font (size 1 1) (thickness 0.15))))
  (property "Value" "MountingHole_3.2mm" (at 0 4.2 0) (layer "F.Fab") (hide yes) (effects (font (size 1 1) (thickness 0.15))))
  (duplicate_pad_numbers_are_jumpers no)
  (pad "" np_thru_hole circle (at 0 0) (size 3.2 3.2) (drill 3.2) (layers "*.Cu" "*.Mask")))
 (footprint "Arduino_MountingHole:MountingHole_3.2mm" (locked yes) (layer "F.Cu") (at 166.04 92.38)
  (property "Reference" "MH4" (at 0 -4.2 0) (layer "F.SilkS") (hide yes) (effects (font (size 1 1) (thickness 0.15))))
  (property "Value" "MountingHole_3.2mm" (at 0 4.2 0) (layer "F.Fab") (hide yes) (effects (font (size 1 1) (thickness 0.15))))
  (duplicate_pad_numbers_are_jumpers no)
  (pad "" np_thru_hole circle (at 0 0) (size 3.2 3.2) (drill 3.2) (layers "*.Cu" "*.Mask")))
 (gr_arc (start 100 47.422) (mid 100.223185 46.883185) (end 100.762 46.66) (stroke (width 0.15) (type solid)) (layer "Edge.Cuts"))
 (gr_line (start 100 99.238) (end 100 47.422) (stroke (width 0.15) (type solid)) (layer "Edge.Cuts"))
 (gr_line (start 100.762 46.66) (end 163.5 46.66) (stroke (width 0.15) (type solid)) (layer "Edge.Cuts"))
 (gr_arc (start 100.762 100) (mid 100.223185 99.776815) (end 100 99.238) (stroke (width 0.15) (type solid)) (layer "Edge.Cuts"))
 (gr_line (start 163.5 46.66) (end 166.04 49.2) (stroke (width 0.15) (type solid)) (layer "Edge.Cuts"))
 (gr_line (start 165.278 100) (end 100.762 100) (stroke (width 0.15) (type solid)) (layer "Edge.Cuts"))
 (gr_line (start 166.04 49.2) (end 166.04 59.36) (stroke (width 0.15) (type solid)) (layer "Edge.Cuts"))
 (gr_line (start 166.04 59.36) (end 168.58 61.9) (stroke (width 0.15) (type solid)) (layer "Edge.Cuts"))
 (gr_line (start 166.04 98.73) (end 166.04 99.238) (stroke (width 0.15) (type solid)) (layer "Edge.Cuts"))
 (gr_arc (start 166.04 99.238) (mid 165.816815 99.776815) (end 165.278 100) (stroke (width 0.15) (type solid)) (layer "Edge.Cuts"))
 (gr_line (start 168.58 61.9) (end 168.58 96.19) (stroke (width 0.15) (type solid)) (layer "Edge.Cuts"))
 (gr_line (start 168.58 96.19) (end 166.04 98.73) (stroke (width 0.15) (type solid)) (layer "Edge.Cuts"))
 (segment (start 138 74.5) (end 138 67.5) (width 0.25) (layer "F.Cu") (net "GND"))
 (segment (start 142 88.96) (end 142 96.28) (width 0.25) (layer "F.Cu") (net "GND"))
 (segment (start 137.5 67) (end 137.5 56.5) (width 0.25) (layer "F.Cu") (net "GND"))
 (segment (start 142 88.96) (end 142 84.66) (width 0.25) (layer "F.Cu") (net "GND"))
 (segment (start 142 84.66) (end 137.84 80.5) (width 0.25) (layer "F.Cu") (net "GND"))
 (segment (start 142 96.28) (end 143.18 97.46) (width 0.25) (layer "F.Cu") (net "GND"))
 (segment (start 137.84 80.5) (end 137.84 74.66) (width 0.25) (layer "F.Cu") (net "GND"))
 (segment (start 138 67.5) (end 137.5 67) (width 0.25) (layer "F.Cu") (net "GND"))
 (segment (start 137.84 74.66) (end 138 74.5) (width 0.25) (layer "F.Cu") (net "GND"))
 (via (at 137.5 56.5) (size 0.6) (drill 0.4) (layers "F.Cu" "B.Cu") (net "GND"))
 (segment (start 137.5 56.5) (end 133.716 56.5) (width 0.25) (layer "B.Cu") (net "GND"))
 (segment (start 133.716 56.5) (end 126.416 49.2) (width 0.25) (layer "B.Cu") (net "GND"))
 (segment (start 130.22 74.66) (end 130.38 74.5) (width 0.25) (layer "F.Cu") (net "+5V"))
 (segment (start 136.92 87.2) (end 130.22 80.5) (width 0.25) (layer "F.Cu") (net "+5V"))
 (segment (start 136.92 88.96) (end 136.92 96.28) (width 0.25) (layer "F.Cu") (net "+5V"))
 (segment (start 132.42 67) (end 132.42 72.46) (width 0.25) (layer "F.Cu") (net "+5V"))
 (segment (start 130.22 80.5) (end 130.22 74.66) (width 0.25) (layer "F.Cu") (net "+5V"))
 (segment (start 130.38 74.5) (end 122.5 74.5) (width 0.25) (layer "F.Cu") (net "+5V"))
 (segment (start 136.92 96.28) (end 138.1 97.46) (width 0.25) (layer "F.Cu") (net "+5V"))
 (segment (start 122.5 74.5) (end 122 74) (width 0.25) (layer "F.Cu") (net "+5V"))
 (segment (start 136.92 88.96) (end 136.92 87.2) (width 0.25) (layer "F.Cu") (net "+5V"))
 (segment (start 132.42 72.46) (end 130.38 74.5) (width 0.25) (layer "F.Cu") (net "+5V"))
 (segment (start 158 77.5) (end 158 94.5) (width 0.25) (layer "F.Cu") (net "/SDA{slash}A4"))
 (segment (start 158 94.5) (end 160.96 97.46) (width 0.25) (layer "F.Cu") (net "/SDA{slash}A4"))
 (via (at 158 77.5) (size 0.6) (drill 0.4) (layers "F.Cu" "B.Cu") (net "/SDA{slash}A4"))
 (segment (start 133.785 61.649) (end 121.336 49.2) (width 0.25) (layer "B.Cu") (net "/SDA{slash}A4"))
 (segment (start 135.46 74.5) (end 133.785 72.825) (width 0.25) (layer "B.Cu") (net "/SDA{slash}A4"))
 (segment (start 138.46 77.5) (end 158 77.5) (width 0.25) (layer "B.Cu") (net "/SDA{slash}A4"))
 (segment (start 135.46 74.5) (end 138.46 77.5) (width 0.25) (layer "B.Cu") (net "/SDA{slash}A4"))
 (segment (start 133.785 72.825) (end 133.785 61.649) (width 0.25) (layer "B.Cu") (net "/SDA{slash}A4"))
 (segment (start 160 78.5) (end 160 93.96) (width 0.25) (layer "F.Cu") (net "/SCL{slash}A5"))
 (segment (start 160 93.96) (end 163.5 97.46) (width 0.25) (layer "F.Cu") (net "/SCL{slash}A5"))
 (via (at 160 78.5) (size 0.6) (drill 0.4) (layers "F.Cu" "B.Cu") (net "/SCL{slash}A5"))
 (segment (start 131 61.404) (end 118.796 49.2) (width 0.25) (layer "B.Cu") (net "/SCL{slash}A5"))
 (segment (start 132.92 74.5) (end 131 72.58) (width 0.25) (layer "B.Cu") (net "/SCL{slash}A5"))
 (segment (start 136.92 78.5) (end 160 78.5) (width 0.25) (layer "B.Cu") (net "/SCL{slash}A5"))
 (segment (start 131 72.58) (end 131 61.404) (width 0.25) (layer "B.Cu") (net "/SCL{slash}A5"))
 (segment (start 132.92 74.5) (end 136.92 78.5) (width 0.25) (layer "B.Cu") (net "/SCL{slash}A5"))
 (segment (start 134.285 79.485) (end 134.285 68.285) (width 0.25) (layer "F.Cu") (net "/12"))
 (segment (start 134.285 68.285) (end 133.595 67.595) (width 0.25) (layer "F.Cu") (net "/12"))
 (segment (start 133.595 51.299) (end 131.496 49.2) (width 0.25) (layer "F.Cu") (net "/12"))
 (segment (start 135.3 80.5) (end 134.285 79.485) (width 0.25) (layer "F.Cu") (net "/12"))
 (segment (start 133.595 67.595) (end 133.595 51.299) (width 0.25) (layer "F.Cu") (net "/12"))
 (segment (start 140.38 80.5) (end 140.38 55.544) (width 0.25) (layer "F.Cu") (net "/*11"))
 (segment (start 140.38 55.544) (end 134.036 49.2) (width 0.25) (layer "F.Cu") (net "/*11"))
 (segment (start 134.96 67) (end 134.96 64.54) (width 0.25) (layer "F.Cu") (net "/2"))
 (segment (start 134.96 64.54) (end 135 64.5) (width 0.25) (layer "F.Cu") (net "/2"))
 (via (at 135 64.5) (size 0.6) (drill 0.4) (layers "F.Cu" "B.Cu") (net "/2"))
 (segment (start 135 64.5) (end 143.12 64.5) (width 0.25) (layer "B.Cu") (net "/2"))
 (segment (start 143.12 64.5) (end 158.42 49.2) (width 0.25) (layer "B.Cu") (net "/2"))
 (segment (start 139.46 87.2) (end 132.76 80.5) (width 0.25) (layer "F.Cu") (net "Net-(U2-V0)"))
 (segment (start 139.46 91.5) (end 139.46 87.2) (width 0.25) (layer "F.Cu") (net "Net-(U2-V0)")))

